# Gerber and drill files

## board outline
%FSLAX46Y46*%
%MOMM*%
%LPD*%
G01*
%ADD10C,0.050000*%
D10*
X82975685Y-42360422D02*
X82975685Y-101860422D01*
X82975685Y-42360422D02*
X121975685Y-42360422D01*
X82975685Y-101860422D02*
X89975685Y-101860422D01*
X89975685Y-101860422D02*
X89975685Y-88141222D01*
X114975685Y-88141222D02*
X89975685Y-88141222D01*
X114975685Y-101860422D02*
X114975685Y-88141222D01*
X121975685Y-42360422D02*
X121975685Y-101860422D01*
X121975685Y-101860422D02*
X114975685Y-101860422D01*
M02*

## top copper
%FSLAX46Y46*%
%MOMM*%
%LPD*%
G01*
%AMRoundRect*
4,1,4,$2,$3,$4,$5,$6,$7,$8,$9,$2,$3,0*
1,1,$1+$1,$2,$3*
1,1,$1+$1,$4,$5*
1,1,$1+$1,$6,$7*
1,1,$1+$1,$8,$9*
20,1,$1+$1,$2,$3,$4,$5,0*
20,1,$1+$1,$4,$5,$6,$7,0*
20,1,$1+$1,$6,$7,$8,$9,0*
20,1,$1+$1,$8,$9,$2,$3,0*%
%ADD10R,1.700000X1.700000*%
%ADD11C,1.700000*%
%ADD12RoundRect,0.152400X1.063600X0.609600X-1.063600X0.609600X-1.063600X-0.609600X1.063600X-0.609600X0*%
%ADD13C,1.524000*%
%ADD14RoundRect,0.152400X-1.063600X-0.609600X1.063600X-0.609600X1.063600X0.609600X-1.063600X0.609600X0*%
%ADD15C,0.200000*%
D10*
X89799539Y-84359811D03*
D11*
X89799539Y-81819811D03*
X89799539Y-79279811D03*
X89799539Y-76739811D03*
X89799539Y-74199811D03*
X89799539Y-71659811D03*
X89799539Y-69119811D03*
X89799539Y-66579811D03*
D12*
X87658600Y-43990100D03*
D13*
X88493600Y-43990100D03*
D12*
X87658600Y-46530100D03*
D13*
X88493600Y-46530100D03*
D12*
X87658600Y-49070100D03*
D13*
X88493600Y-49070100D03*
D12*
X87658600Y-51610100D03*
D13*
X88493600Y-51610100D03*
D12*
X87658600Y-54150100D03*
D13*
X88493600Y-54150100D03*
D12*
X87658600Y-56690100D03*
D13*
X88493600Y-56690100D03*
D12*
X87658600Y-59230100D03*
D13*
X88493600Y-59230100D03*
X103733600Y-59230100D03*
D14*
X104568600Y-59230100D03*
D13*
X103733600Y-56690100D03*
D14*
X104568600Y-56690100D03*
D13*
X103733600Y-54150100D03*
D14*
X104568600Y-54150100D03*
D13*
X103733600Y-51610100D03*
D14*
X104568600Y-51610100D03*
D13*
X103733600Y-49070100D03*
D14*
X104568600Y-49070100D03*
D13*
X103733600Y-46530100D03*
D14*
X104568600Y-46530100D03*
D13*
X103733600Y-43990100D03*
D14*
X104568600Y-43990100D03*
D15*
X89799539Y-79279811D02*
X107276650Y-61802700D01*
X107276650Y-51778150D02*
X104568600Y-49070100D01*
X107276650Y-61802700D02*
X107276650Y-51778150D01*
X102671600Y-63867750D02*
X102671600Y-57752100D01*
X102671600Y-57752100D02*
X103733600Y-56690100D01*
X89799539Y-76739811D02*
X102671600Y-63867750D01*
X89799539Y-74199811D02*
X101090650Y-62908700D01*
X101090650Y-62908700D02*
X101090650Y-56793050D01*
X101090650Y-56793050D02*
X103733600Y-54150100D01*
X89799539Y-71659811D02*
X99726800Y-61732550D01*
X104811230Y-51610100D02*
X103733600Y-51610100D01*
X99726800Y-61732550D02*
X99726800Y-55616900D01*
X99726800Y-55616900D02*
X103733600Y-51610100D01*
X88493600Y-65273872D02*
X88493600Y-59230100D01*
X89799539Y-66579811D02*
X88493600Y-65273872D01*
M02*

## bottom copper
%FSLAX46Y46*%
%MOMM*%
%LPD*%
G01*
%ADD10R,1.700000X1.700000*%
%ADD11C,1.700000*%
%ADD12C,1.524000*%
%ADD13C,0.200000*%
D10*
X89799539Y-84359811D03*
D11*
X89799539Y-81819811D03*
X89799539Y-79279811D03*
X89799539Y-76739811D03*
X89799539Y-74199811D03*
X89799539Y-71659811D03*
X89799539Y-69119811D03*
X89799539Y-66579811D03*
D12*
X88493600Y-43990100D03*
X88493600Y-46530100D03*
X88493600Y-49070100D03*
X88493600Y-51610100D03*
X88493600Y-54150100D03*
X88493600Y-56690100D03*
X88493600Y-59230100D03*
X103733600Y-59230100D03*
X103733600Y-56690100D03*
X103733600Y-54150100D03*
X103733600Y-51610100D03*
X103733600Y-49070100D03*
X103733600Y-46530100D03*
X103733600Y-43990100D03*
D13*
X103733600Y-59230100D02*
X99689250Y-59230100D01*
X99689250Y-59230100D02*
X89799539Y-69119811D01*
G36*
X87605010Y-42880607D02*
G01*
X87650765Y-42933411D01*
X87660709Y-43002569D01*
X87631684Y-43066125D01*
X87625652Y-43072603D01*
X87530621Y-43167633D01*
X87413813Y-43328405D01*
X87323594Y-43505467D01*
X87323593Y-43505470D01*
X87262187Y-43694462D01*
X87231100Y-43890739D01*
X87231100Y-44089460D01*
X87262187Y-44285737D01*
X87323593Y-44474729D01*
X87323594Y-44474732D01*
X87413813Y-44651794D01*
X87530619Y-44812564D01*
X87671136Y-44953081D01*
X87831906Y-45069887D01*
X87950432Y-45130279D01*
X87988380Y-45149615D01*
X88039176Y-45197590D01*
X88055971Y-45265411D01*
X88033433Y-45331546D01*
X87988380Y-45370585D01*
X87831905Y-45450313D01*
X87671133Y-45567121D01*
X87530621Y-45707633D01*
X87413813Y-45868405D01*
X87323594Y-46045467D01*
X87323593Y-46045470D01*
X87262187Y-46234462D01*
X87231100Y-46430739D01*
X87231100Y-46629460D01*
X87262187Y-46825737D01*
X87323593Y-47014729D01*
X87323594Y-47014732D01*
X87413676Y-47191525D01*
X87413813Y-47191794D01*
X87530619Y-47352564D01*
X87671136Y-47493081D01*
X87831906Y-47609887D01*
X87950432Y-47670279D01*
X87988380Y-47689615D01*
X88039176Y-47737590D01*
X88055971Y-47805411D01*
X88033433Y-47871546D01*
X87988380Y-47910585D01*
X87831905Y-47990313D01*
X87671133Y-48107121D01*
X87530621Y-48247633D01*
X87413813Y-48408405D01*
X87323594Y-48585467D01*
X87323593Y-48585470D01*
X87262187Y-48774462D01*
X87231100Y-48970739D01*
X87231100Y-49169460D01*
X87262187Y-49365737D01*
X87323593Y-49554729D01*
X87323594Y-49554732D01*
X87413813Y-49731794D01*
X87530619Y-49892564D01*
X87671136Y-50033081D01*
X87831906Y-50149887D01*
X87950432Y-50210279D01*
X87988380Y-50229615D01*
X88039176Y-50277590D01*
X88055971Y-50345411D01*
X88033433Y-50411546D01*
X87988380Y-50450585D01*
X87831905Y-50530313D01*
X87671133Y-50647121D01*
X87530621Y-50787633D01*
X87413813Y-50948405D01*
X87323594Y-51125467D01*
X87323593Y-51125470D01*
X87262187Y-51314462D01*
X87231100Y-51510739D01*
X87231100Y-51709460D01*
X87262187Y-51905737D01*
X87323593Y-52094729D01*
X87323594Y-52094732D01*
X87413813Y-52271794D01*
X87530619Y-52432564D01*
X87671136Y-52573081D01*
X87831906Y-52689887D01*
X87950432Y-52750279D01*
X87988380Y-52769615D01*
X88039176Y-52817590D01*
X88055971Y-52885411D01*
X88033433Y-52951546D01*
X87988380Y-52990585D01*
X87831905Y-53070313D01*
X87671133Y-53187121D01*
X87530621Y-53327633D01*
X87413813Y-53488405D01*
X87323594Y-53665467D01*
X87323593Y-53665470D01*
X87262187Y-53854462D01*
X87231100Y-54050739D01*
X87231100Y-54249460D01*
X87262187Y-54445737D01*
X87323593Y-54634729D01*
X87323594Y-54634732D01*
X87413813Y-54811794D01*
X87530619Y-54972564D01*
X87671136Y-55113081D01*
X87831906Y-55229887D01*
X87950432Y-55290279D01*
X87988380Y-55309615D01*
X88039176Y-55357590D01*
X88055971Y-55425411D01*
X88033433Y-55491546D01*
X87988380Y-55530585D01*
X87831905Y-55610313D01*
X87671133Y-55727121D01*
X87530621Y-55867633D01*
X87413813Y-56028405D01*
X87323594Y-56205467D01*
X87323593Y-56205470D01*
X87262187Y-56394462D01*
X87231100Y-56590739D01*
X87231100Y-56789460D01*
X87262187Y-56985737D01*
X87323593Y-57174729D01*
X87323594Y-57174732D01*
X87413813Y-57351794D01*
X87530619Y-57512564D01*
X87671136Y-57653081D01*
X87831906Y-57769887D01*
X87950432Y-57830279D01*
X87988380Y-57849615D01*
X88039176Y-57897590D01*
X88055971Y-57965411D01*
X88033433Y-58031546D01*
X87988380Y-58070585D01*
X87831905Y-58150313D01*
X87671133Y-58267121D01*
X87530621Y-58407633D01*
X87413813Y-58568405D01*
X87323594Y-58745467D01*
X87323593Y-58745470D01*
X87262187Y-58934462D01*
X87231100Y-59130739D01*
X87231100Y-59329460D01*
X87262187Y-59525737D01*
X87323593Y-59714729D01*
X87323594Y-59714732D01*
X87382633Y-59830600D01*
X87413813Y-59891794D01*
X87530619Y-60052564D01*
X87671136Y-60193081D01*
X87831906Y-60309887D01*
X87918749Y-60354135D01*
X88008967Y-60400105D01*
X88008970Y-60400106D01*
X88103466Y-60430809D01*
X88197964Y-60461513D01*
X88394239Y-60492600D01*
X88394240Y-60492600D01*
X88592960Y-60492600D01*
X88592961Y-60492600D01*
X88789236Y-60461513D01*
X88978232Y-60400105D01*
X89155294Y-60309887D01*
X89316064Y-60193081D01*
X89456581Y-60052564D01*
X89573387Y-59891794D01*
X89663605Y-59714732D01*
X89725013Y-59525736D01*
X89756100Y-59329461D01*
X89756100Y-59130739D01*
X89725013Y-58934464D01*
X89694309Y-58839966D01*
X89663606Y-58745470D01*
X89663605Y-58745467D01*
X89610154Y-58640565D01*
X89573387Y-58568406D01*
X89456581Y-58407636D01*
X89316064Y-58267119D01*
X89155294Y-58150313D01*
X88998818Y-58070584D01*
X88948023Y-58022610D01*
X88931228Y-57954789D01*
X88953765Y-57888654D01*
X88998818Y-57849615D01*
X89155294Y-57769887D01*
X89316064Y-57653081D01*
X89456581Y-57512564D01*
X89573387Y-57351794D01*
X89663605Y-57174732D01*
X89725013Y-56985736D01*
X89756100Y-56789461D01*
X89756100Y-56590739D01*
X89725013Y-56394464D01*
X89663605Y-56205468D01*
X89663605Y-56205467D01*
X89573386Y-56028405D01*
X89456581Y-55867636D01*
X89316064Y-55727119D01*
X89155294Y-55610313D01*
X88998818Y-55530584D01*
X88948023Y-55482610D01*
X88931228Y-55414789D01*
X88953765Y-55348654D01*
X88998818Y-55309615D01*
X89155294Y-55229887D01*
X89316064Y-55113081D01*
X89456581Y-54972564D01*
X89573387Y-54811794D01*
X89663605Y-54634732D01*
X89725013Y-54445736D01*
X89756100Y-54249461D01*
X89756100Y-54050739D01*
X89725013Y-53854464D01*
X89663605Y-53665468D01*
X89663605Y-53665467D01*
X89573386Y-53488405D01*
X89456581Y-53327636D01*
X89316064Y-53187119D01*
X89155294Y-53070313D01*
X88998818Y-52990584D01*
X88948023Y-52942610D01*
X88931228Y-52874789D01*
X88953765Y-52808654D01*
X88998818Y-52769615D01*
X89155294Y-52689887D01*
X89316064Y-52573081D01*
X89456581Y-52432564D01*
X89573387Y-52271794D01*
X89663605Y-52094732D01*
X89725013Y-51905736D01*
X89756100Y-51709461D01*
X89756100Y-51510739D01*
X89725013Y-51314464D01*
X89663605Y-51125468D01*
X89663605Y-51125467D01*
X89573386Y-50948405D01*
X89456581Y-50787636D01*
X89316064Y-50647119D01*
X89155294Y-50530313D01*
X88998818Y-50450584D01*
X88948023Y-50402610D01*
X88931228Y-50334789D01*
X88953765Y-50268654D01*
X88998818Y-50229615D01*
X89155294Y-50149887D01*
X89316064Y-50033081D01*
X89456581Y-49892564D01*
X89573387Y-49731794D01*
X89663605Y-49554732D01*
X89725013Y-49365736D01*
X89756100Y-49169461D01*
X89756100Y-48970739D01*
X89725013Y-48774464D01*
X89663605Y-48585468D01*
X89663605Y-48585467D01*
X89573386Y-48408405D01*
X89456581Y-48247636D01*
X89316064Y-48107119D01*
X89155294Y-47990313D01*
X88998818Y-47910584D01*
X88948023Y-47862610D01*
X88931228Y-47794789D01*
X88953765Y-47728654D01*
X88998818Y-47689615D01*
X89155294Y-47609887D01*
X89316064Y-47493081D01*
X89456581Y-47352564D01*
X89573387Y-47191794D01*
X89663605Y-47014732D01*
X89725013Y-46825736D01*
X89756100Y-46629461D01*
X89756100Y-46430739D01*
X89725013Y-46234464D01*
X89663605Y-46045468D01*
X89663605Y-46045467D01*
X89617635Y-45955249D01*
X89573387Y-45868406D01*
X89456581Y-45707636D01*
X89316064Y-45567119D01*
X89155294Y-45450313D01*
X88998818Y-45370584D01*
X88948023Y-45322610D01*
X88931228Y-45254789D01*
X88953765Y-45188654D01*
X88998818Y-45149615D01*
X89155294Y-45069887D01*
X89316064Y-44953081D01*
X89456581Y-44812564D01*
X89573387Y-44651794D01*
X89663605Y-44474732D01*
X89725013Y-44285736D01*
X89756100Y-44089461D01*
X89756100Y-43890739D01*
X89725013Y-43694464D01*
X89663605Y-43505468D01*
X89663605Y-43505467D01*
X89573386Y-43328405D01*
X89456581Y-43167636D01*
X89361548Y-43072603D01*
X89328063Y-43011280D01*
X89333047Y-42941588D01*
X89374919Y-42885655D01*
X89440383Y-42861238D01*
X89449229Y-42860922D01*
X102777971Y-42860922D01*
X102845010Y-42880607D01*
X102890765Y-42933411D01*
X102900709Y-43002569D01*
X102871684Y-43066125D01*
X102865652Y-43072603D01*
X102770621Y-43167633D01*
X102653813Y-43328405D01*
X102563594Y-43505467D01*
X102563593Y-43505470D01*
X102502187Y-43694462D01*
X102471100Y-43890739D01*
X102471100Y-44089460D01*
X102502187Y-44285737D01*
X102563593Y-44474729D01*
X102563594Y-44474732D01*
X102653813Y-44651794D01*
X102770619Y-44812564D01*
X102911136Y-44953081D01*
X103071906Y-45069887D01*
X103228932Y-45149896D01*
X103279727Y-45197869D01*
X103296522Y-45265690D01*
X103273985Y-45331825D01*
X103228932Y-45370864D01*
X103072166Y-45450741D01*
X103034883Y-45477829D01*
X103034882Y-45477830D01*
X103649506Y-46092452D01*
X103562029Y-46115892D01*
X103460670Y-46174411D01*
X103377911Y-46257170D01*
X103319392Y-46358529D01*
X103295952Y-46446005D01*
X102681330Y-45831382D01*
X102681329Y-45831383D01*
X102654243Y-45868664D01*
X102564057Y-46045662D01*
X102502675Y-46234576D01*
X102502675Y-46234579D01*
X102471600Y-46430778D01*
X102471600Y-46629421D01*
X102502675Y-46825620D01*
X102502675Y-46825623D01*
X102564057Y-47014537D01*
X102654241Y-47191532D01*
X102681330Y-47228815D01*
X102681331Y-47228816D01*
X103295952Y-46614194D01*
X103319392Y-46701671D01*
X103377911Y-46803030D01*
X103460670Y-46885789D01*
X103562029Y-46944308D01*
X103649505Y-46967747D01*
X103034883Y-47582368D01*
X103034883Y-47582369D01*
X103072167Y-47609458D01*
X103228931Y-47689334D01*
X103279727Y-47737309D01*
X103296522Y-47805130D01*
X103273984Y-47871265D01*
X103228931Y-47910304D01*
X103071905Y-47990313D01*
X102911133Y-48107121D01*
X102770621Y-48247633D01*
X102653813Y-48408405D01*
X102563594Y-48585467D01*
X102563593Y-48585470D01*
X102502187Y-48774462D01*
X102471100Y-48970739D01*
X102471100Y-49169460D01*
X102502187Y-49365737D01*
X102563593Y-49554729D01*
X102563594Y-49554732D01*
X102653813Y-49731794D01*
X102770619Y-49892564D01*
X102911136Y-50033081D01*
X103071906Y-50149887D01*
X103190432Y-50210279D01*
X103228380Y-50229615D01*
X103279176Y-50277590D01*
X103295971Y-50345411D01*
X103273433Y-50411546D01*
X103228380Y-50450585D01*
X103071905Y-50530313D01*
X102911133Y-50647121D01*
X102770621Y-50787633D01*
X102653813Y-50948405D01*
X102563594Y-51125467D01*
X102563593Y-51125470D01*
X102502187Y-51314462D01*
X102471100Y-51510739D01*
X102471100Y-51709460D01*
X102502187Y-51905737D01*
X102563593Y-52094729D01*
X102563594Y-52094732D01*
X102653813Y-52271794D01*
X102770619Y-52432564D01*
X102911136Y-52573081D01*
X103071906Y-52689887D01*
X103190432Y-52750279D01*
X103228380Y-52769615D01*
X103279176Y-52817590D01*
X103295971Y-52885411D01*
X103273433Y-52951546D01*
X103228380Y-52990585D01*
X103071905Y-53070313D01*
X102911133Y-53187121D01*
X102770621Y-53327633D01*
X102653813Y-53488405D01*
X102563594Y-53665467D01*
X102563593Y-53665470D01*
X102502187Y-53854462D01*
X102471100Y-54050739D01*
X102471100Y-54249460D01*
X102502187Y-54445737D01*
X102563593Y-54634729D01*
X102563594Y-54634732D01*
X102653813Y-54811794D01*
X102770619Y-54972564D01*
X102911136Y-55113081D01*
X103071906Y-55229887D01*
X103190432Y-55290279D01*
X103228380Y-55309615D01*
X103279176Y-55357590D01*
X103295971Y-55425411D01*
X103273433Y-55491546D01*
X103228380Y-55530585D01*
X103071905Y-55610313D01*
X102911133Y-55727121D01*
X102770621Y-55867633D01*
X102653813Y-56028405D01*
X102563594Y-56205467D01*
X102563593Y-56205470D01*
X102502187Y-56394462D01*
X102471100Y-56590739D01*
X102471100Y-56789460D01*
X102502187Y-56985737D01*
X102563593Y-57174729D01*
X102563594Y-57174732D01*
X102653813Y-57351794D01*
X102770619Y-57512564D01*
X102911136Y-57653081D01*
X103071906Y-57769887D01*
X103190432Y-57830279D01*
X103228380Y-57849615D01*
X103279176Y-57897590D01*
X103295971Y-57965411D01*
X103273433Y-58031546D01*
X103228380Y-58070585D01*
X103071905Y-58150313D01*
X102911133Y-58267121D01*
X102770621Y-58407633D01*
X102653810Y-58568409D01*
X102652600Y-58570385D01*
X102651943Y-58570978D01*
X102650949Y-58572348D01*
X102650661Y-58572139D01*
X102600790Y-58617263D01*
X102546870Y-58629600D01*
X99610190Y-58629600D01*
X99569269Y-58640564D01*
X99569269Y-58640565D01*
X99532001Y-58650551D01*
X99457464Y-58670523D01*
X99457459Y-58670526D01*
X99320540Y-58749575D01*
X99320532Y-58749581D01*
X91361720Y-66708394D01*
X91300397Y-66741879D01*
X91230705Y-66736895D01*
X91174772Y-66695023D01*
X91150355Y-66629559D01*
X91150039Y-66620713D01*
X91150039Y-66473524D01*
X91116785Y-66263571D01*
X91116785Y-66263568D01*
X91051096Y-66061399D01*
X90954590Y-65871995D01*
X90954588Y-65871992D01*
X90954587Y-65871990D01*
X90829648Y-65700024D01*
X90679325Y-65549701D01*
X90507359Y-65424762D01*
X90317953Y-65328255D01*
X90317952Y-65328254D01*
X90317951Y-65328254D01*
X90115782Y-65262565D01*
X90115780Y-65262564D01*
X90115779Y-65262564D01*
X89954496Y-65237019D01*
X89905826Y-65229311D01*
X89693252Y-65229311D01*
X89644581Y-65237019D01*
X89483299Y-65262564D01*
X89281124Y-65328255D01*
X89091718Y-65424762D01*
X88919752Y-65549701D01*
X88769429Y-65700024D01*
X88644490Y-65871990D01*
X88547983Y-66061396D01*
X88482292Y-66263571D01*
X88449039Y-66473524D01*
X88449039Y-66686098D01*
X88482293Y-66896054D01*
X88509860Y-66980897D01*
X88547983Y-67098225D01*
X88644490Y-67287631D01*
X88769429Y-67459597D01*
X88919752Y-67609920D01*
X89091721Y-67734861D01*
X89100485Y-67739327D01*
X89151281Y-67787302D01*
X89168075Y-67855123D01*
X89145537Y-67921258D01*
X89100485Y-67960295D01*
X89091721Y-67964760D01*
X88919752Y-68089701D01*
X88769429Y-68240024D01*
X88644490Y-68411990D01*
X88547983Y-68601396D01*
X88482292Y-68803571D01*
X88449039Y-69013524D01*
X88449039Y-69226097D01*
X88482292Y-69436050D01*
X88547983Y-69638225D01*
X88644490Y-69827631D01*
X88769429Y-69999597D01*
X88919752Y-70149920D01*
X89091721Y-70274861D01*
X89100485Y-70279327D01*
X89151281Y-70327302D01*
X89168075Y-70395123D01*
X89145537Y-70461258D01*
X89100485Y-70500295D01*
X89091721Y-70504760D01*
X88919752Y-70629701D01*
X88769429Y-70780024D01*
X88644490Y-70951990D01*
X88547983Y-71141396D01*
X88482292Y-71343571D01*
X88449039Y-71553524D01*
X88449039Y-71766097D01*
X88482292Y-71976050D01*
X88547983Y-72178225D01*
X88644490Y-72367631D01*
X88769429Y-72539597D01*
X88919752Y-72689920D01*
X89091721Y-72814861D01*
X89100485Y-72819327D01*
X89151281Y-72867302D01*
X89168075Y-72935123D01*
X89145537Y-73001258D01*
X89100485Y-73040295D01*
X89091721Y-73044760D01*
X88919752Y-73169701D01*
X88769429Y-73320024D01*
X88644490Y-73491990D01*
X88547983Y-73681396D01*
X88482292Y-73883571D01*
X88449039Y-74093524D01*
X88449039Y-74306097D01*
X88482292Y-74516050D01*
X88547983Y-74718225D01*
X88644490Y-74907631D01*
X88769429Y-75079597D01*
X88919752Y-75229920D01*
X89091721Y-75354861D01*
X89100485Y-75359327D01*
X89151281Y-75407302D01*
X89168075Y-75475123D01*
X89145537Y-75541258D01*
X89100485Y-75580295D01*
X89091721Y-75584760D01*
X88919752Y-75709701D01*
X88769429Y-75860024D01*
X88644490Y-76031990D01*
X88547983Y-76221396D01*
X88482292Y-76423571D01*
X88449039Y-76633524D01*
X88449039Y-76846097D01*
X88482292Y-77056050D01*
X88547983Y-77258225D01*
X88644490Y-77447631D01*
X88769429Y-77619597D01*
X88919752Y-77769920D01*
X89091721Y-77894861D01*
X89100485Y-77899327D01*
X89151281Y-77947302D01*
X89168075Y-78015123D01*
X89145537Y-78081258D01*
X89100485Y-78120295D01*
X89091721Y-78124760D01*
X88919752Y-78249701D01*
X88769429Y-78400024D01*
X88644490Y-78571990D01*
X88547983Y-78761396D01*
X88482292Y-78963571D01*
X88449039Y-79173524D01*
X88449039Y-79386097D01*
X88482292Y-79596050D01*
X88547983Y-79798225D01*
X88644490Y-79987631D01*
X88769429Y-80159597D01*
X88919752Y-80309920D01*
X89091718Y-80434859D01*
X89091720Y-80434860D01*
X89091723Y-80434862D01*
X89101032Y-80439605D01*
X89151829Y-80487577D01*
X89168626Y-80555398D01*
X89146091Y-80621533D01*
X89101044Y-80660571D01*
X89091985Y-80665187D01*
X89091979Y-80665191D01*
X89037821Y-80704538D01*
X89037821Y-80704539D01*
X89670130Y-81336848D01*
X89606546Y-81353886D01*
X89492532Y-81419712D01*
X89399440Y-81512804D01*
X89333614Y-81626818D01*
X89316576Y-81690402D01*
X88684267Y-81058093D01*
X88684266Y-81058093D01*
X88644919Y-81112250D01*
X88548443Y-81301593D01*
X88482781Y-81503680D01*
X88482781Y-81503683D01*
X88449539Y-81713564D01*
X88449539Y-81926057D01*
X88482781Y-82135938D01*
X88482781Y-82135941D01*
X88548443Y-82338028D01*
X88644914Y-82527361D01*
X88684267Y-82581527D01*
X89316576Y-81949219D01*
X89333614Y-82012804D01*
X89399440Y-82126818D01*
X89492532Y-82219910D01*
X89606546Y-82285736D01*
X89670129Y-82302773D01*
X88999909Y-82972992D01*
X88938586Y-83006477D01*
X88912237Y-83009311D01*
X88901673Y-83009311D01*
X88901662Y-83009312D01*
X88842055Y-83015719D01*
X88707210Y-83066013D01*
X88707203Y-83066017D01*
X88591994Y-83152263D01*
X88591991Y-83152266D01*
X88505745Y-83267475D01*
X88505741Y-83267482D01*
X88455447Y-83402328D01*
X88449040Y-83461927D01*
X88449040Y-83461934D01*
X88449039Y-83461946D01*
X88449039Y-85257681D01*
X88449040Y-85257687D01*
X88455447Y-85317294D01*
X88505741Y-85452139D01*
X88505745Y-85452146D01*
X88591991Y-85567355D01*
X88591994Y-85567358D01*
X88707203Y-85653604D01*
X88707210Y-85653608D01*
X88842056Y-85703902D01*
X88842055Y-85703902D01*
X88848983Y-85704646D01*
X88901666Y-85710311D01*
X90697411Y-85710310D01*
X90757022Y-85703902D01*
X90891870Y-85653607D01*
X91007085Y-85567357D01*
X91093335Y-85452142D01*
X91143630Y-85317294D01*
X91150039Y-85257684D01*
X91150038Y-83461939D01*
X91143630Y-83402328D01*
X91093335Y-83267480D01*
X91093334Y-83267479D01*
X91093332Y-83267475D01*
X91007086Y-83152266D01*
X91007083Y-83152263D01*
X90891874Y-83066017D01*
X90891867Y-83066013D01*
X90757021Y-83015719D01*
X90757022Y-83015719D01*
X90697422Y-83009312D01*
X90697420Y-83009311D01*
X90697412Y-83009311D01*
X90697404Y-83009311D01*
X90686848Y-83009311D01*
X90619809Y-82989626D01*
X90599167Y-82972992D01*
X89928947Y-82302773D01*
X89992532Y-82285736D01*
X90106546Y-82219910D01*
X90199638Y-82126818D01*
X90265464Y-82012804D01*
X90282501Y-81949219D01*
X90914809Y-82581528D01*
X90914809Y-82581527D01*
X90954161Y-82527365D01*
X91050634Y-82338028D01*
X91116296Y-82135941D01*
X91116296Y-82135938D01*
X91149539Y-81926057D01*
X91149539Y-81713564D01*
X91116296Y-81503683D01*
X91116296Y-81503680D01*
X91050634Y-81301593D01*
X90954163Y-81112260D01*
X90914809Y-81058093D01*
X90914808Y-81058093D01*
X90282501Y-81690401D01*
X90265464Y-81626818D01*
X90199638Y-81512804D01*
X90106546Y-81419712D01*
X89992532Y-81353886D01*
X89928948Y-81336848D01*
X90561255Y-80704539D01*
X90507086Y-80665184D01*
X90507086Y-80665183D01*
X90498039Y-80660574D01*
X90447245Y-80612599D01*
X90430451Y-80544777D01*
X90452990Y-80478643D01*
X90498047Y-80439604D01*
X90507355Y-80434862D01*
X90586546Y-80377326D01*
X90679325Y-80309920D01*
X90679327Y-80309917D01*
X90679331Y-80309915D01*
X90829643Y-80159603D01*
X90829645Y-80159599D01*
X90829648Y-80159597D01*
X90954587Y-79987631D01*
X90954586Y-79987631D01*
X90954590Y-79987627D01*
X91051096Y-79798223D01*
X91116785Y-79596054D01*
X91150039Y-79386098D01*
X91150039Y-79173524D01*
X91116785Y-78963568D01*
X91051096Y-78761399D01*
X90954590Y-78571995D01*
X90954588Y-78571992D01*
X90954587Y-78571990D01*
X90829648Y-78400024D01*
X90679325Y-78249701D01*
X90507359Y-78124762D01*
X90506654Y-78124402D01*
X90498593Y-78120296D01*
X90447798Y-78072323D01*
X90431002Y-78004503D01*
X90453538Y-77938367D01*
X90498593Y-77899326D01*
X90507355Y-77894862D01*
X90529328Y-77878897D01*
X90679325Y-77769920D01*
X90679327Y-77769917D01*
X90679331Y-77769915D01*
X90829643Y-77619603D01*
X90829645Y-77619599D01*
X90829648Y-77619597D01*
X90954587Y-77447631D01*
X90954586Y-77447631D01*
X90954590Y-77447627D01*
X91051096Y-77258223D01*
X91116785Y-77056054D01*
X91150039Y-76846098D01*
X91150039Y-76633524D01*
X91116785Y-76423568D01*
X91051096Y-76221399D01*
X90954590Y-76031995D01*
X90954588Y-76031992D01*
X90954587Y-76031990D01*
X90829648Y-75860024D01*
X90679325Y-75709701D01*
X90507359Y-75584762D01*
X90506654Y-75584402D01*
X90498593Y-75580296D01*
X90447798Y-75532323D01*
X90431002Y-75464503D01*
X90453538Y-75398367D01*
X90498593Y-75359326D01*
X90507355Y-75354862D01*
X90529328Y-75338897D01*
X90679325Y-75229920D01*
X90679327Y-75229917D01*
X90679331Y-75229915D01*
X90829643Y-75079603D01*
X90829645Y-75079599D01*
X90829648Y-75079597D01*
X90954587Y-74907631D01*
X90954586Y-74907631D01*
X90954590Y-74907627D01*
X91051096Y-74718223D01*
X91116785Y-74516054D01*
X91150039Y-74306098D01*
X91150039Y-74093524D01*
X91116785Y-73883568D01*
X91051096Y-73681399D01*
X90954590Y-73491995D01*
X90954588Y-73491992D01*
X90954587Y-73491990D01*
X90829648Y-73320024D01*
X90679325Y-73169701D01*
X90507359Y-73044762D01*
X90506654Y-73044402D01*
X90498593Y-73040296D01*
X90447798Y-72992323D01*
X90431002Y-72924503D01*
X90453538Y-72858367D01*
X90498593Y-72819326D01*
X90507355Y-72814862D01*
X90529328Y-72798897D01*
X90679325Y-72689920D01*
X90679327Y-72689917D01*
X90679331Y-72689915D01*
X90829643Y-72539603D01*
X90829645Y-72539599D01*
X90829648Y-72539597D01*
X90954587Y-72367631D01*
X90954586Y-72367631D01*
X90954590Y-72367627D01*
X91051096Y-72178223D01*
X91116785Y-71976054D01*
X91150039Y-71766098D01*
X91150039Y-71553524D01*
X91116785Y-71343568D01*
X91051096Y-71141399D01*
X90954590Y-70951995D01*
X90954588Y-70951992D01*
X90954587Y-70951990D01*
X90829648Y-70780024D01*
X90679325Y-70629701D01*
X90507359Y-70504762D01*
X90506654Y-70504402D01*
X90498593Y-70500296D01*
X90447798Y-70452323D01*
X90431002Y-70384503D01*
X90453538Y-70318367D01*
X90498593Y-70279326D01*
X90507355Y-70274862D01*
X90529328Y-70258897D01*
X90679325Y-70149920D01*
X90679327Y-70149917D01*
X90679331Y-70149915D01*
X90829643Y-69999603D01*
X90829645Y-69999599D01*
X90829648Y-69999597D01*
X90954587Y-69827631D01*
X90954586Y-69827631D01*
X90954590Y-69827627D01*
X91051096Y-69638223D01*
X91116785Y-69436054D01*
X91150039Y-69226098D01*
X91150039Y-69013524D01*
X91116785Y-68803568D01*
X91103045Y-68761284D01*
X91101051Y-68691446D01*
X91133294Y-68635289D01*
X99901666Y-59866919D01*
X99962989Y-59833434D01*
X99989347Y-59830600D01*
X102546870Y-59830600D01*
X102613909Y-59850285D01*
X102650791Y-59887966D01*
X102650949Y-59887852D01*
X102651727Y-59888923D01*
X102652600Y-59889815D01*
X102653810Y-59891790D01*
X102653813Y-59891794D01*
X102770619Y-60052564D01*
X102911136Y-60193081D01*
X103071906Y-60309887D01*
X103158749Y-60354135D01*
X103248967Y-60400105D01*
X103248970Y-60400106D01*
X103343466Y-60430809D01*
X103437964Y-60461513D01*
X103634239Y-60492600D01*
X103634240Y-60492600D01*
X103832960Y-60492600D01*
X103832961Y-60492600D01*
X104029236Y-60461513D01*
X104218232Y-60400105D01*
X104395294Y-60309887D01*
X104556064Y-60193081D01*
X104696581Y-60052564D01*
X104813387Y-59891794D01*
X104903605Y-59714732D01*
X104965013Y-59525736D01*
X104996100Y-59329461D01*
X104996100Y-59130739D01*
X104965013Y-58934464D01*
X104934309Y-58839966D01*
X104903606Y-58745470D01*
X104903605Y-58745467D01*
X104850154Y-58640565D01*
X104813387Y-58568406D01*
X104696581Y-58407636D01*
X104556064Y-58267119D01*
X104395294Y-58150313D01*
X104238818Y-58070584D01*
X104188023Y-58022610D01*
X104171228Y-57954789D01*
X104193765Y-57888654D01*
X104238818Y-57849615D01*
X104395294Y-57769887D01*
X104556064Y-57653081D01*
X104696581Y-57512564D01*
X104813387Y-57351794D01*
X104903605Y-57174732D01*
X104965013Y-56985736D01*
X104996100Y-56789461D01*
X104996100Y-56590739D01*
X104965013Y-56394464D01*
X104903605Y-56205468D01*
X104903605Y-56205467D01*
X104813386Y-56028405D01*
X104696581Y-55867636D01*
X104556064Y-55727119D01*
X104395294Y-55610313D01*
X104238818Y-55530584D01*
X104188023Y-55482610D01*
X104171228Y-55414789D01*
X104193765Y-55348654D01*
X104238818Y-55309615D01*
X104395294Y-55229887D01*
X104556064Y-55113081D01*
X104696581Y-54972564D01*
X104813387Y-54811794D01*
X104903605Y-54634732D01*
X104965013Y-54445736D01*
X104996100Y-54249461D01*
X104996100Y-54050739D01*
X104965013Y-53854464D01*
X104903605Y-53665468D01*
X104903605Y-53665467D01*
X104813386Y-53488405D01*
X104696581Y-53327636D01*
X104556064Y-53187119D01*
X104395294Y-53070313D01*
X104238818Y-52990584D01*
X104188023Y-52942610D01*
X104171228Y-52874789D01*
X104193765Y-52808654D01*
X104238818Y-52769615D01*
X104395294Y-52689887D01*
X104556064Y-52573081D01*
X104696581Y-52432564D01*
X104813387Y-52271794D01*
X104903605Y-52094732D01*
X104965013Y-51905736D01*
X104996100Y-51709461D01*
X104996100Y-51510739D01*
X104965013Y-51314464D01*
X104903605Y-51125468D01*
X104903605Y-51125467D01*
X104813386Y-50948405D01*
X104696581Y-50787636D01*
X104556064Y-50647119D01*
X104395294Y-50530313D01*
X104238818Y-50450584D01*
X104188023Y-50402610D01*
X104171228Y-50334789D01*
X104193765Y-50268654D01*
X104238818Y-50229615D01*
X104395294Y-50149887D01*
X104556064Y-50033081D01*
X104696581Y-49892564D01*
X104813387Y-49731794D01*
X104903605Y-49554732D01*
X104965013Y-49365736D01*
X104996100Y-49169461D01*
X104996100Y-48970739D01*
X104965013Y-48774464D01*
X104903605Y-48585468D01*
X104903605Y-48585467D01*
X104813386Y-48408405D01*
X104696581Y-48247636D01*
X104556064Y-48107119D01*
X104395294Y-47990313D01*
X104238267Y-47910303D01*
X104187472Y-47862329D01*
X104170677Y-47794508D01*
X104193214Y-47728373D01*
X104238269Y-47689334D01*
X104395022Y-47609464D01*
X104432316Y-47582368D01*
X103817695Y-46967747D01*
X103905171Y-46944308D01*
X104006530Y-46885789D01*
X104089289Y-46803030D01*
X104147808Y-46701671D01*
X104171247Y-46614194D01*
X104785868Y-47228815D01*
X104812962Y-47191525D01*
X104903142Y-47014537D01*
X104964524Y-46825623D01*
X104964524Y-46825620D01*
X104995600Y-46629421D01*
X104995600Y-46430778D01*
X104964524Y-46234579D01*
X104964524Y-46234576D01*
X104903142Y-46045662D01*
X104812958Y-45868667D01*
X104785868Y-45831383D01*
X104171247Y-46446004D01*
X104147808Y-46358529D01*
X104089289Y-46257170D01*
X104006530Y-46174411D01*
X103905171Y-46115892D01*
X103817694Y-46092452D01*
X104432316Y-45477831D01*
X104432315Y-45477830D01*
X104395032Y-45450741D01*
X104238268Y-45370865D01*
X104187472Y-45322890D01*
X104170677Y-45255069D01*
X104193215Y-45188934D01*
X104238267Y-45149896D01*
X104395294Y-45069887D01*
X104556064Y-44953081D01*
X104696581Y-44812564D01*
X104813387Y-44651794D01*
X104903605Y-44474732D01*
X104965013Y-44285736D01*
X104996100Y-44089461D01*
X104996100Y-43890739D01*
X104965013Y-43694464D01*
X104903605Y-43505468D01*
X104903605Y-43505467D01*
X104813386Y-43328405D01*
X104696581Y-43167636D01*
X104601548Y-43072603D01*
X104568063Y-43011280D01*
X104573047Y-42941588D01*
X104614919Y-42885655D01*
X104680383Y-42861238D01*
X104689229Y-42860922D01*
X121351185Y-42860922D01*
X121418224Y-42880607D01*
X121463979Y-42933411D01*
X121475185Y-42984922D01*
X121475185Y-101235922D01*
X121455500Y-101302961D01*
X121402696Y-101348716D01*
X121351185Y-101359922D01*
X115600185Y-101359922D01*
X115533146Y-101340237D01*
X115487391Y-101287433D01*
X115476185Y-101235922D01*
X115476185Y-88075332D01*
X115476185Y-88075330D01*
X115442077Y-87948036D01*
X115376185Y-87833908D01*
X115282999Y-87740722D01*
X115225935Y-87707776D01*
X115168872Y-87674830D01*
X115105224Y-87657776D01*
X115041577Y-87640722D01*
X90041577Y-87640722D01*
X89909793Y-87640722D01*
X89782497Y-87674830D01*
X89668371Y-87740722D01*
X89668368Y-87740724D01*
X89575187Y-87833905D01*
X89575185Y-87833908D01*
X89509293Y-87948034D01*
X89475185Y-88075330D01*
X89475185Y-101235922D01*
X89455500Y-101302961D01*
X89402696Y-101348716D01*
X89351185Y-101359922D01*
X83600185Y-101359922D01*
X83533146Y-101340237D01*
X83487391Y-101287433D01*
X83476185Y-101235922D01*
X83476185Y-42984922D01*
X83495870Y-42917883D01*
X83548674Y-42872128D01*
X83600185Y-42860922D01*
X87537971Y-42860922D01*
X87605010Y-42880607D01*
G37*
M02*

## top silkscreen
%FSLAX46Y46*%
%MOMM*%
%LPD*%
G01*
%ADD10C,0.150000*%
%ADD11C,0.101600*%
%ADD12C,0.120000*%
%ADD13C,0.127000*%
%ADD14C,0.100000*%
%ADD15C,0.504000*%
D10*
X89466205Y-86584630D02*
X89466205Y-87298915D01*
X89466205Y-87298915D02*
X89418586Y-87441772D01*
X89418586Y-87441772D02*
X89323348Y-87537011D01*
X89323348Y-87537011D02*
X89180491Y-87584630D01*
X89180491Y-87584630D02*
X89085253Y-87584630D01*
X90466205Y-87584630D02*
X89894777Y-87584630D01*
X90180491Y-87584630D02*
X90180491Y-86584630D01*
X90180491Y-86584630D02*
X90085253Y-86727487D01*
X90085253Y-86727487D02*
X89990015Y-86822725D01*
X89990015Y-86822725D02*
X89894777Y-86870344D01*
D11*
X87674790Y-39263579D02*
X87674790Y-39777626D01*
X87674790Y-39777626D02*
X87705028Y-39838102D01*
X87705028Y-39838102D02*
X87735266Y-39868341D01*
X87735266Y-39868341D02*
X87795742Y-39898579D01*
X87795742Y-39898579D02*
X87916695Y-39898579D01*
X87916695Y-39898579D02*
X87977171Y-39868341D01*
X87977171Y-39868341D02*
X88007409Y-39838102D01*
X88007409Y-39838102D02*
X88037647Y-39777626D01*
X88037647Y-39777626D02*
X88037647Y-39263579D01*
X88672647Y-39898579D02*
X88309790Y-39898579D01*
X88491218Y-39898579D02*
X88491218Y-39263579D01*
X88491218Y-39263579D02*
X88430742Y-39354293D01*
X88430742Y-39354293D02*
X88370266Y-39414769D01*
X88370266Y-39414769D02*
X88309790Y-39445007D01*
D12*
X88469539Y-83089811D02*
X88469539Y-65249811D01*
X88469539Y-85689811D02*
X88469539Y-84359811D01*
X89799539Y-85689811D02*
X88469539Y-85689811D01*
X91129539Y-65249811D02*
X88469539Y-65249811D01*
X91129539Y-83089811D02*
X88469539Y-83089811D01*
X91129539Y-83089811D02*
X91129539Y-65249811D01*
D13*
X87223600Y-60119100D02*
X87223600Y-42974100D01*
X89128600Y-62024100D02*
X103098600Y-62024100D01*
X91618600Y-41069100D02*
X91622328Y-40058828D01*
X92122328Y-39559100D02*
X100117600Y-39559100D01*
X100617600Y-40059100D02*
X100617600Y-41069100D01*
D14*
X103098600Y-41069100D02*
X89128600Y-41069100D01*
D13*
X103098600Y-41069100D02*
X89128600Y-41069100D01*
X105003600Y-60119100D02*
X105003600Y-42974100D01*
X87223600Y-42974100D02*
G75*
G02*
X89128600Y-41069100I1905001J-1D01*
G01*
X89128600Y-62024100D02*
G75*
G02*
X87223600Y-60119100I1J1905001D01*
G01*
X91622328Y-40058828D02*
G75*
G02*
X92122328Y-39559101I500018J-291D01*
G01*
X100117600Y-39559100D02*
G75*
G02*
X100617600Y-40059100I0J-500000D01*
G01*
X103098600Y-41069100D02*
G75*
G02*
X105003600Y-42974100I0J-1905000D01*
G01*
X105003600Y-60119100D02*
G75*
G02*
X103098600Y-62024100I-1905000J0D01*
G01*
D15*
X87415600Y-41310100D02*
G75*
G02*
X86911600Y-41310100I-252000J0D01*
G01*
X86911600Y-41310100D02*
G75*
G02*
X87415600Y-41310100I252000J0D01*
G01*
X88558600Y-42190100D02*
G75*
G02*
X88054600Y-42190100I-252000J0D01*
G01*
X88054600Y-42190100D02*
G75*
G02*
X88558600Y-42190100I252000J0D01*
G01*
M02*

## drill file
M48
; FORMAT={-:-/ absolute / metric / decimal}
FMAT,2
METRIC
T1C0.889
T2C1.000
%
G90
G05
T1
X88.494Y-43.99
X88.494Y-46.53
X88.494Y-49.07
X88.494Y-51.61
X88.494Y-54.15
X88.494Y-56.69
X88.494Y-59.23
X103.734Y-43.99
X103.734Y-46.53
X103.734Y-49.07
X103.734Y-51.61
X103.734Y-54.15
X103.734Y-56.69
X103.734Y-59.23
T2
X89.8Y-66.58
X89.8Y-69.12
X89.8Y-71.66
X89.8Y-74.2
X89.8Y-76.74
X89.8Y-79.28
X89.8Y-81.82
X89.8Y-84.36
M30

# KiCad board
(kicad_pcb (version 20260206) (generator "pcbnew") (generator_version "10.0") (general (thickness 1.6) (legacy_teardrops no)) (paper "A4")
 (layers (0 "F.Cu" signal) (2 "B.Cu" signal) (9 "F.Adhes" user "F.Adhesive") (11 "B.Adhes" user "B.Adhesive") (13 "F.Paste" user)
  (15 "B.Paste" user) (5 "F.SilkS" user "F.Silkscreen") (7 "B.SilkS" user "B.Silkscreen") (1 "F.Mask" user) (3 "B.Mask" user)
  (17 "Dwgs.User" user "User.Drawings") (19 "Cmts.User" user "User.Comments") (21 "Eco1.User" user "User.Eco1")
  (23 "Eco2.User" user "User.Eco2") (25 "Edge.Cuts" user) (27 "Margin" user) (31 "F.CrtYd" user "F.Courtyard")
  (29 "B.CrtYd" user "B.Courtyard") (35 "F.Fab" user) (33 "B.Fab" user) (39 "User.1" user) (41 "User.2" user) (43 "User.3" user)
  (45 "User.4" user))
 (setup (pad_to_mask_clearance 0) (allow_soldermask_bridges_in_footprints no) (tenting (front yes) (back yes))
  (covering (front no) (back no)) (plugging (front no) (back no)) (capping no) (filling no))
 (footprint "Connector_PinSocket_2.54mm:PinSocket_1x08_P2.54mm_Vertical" (layer "F.Cu") (at 89.799539 84.359811 180)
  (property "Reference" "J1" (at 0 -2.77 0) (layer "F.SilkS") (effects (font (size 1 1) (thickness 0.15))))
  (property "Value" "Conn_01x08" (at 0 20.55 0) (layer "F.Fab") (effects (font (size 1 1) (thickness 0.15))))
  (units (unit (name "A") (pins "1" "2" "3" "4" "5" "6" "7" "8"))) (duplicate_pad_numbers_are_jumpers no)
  (fp_line (start 1.33 1.27) (end 1.33 19.11) (stroke (width 0.12) (type solid)) (layer "F.SilkS"))
  (fp_line (start 1.33 -1.33) (end 1.33 0) (stroke (width 0.12) (type solid)) (layer "F.SilkS"))
  (fp_line (start 0 -1.33) (end 1.33 -1.33) (stroke (width 0.12) (type solid)) (layer "F.SilkS"))
  (fp_line (start -1.33 19.11) (end 1.33 19.11) (stroke (width 0.12) (type solid)) (layer "F.SilkS"))
  (fp_line (start -1.33 1.27) (end 1.33 1.27) (stroke (width 0.12) (type solid)) (layer "F.SilkS"))
  (fp_line (start -1.33 1.27) (end -1.33 19.11) (stroke (width 0.12) (type solid)) (layer "F.SilkS"))
  (pad "1" thru_hole rect (at 0 0 180) (size 1.7 1.7) (drill 1) (layers "*.Cu" "*.Mask") (remove_unused_layers no) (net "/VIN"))
  (pad "2" thru_hole circle (at 0 2.54 180) (size 1.7 1.7) (drill 1) (layers "*.Cu" "*.Mask") (remove_unused_layers no) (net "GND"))
  (pad "3" thru_hole circle (at 0 5.08 180) (size 1.7 1.7) (drill 1) (layers "*.Cu" "*.Mask") (remove_unused_layers no) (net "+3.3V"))
  (pad "4" thru_hole circle (at 0 7.62 180) (size 1.7 1.7) (drill 1) (layers "*.Cu" "*.Mask") (remove_unused_layers no) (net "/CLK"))
  (pad "5" thru_hole circle (at 0 10.16 180) (size 1.7 1.7) (drill 1) (layers "*.Cu" "*.Mask") (remove_unused_layers no) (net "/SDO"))
  (pad "6" thru_hole circle (at 0 12.7 180) (size 1.7 1.7) (drill 1) (layers "*.Cu" "*.Mask") (remove_unused_layers no) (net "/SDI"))
  (pad "7" thru_hole circle (at 0 15.24 180) (size 1.7 1.7) (drill 1) (layers "*.Cu" "*.Mask") (remove_unused_layers no) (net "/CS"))
  (pad "8" thru_hole circle (at 0 17.78 180) (size 1.7 1.7) (drill 1) (layers "*.Cu" "*.Mask") (remove_unused_layers no) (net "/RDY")))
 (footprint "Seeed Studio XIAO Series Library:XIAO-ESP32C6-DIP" (layer "F.Cu") (at 96.1586 51.6101)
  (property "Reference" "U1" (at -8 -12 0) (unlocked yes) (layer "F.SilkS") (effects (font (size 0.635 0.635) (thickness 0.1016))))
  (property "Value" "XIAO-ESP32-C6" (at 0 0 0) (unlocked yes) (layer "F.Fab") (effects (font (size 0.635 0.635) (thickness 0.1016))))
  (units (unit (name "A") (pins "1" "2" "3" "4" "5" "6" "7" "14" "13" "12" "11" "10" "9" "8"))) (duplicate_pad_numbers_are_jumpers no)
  (fp_line (start -8.935 8.509) (end -8.935 -8.636) (stroke (width 0.127) (type solid)) (layer "F.SilkS"))
  (fp_line (start -7.03 10.414) (end 6.94 10.414) (stroke (width 0.127) (type solid)) (layer "F.SilkS"))
  (fp_line (start -4.54 -10.541) (end -4.536272 -11.551272) (stroke (width 0.127) (type solid)) (layer "F.SilkS"))
  (fp_line (start -4.036272 -12.051) (end 3.959 -12.051) (stroke (width 0.127) (type solid)) (layer "F.SilkS"))
  (fp_line (start 4.459 -11.551) (end 4.459 -10.541) (stroke (width 0.127) (type solid)) (layer "F.SilkS"))
  (fp_line (start 6.94 -10.541) (end -7.03 -10.541) (stroke (width 0.1) (type solid)) (layer "F.SilkS"))
  (fp_line (start 6.94 -10.541) (end -7.03 -10.541) (stroke (width 0.127) (type solid)) (layer "F.SilkS"))
  (fp_line (start 8.845 8.509) (end 8.845 -8.636) (stroke (width 0.127) (type solid)) (layer "F.SilkS"))
  (fp_arc (start -8.935 -8.636) (mid -8.377038 -9.983038) (end -7.03 -10.541) (stroke (width 0.127) (type solid)) (layer "F.SilkS"))
  (fp_arc (start -7.03 10.414) (mid -8.377038 9.856038) (end -8.935 8.509) (stroke (width 0.127) (type solid)) (layer "F.SilkS"))
  (fp_arc (start -4.536272 -11.551272) (mid -4.389728 -11.90464) (end -4.036272 -12.051) (stroke (width 0.127) (type default))
   (layer "F.SilkS"))
  (fp_arc (start 3.959 -12.051) (mid 4.312553 -11.904553) (end 4.459 -11.551) (stroke (width 0.127) (type default)) (layer "F.SilkS"))
  (fp_arc (start 6.94 -10.541) (mid 8.287038 -9.983038) (end 8.845 -8.636) (stroke (width 0.127) (type solid)) (layer "F.SilkS"))
  (fp_arc (start 8.845 8.509) (mid 8.287038 9.856038) (end 6.94 10.414) (stroke (width 0.127) (type solid)) (layer "F.SilkS"))
  (fp_circle (center -8.995 -10.3) (end -8.995 -10.554) (stroke (width 0.5) (type solid)) (fill yes) (layer "F.SilkS"))
  (fp_circle (center -7.852 -9.42) (end -7.852 -9.674) (stroke (width 0.5) (type solid)) (fill yes) (layer "F.SilkS"))
  (pad "1" smd roundrect (at -8.5 -7.62 180) (size 2.432 1.524) (layers "F.Cu" "F.Mask") (roundrect_rratio 0.1)
   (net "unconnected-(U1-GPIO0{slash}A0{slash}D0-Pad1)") (thermal_bridge_angle 45))
  (pad "1" thru_hole circle (at -7.665 -7.62 180) (size 1.524 1.524) (drill 0.889) (layers "*.Cu" "*.Mask") (remove_unused_layers no)
   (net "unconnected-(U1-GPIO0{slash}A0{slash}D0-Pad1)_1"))
  (pad "2" smd roundrect (at -8.5 -5.08 180) (size 2.432 1.524) (layers "F.Cu" "F.Mask") (roundrect_rratio 0.1)
   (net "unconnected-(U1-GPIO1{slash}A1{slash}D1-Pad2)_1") (thermal_bridge_angle 45))
  (pad "2" thru_hole circle (at -7.665 -5.08 180) (size 1.524 1.524) (drill 0.889) (layers "*.Cu" "*.Mask") (remove_unused_layers no)
   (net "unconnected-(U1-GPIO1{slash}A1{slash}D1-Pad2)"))
  (pad "3" smd roundrect (at -8.5 -2.54 180) (size 2.432 1.524) (layers "F.Cu" "F.Mask") (roundrect_rratio 0.1)
   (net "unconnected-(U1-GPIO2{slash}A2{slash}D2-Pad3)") (thermal_bridge_angle 45))
  (pad "3" thru_hole circle (at -7.665 -2.54 180) (size 1.524 1.524) (drill 0.889) (layers "*.Cu" "*.Mask") (remove_unused_layers no)
   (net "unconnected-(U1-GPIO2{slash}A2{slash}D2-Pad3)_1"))
  (pad "4" smd roundrect (at -8.5 0 180) (size 2.432 1.524) (layers "F.Cu" "F.Mask") (roundrect_rratio 0.1)
   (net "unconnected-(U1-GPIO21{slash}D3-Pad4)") (thermal_bridge_angle 45))
  (pad "4" thru_hole circle (at -7.665 0 180) (size 1.524 1.524) (drill 0.889) (layers "*.Cu" "*.Mask") (remove_unused_layers no)
   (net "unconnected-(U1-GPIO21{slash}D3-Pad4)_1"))
  (pad "5" smd roundrect (at -8.5 2.54 180) (size 2.432 1.524) (layers "F.Cu" "F.Mask") (roundrect_rratio 0.1)
   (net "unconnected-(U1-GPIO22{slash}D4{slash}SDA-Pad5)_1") (thermal_bridge_angle 45))
  (pad "5" thru_hole circle (at -7.665 2.54 180) (size 1.524 1.524) (drill 0.889) (layers "*.Cu" "*.Mask") (remove_unused_layers no)
   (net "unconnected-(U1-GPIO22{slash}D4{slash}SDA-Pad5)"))
  (pad "6" smd roundrect (at -8.5 5.08 180) (size 2.432 1.524) (layers "F.Cu" "F.Mask") (roundrect_rratio 0.1)
   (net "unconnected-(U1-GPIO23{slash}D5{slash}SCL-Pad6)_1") (thermal_bridge_angle 45))
  (pad "6" thru_hole circle (at -7.665 5.08 180) (size 1.524 1.524) (drill 0.889) (layers "*.Cu" "*.Mask") (remove_unused_layers no)
   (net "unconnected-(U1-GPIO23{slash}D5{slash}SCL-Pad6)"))
  (pad "7" smd roundrect (at -8.5 7.62 180) (size 2.432 1.524) (layers "F.Cu" "F.Mask") (roundrect_rratio 0.1) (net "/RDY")
   (thermal_bridge_angle 45))
  (pad "7" thru_hole circle (at -7.665 7.62 180) (size 1.524 1.524) (drill 0.889) (layers "*.Cu" "*.Mask") (remove_unused_layers no)
   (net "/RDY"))
  (pad "8" thru_hole circle (at 7.575 7.62) (size 1.524 1.524) (drill 0.889) (layers "*.Cu" "*.Mask") (remove_unused_layers no) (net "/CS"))
  (pad "8" smd roundrect (at 8.41 7.62) (size 2.432 1.524) (layers "F.Cu" "F.Mask") (roundrect_rratio 0.1) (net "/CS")
   (thermal_bridge_angle 45))
  (pad "9" thru_hole circle (at 7.575 5.08) (size 1.524 1.524) (drill 0.889) (layers "*.Cu" "*.Mask") (remove_unused_layers no) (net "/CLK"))
  (pad "9" smd roundrect (at 8.41 5.08) (size 2.432 1.524) (layers "F.Cu" "F.Mask") (roundrect_rratio 0.1) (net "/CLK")
   (thermal_bridge_angle 45))
  (pad "10" thru_hole circle (at 7.575 2.54) (size 1.524 1.524) (drill 0.889) (layers "*.Cu" "*.Mask") (remove_unused_layers no)
   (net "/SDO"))
  (pad "10" smd roundrect (at 8.41 2.54) (size 2.432 1.524) (layers "F.Cu" "F.Mask") (roundrect_rratio 0.1) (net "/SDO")
   (thermal_bridge_angle 45))
  (pad "11" thru_hole circle (at 7.575 0) (size 1.524 1.524) (drill 0.889) (layers "*.Cu" "*.Mask") (remove_unused_layers no) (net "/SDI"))
  (pad "11" smd roundrect (at 8.41 0) (size 2.432 1.524) (layers "F.Cu" "F.Mask") (roundrect_rratio 0.1) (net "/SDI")
   (thermal_bridge_angle 45))
  (pad "12" thru_hole circle (at 7.575 -2.54) (size 1.524 1.524) (drill 0.889) (layers "*.Cu" "*.Mask") (remove_unused_layers no)
   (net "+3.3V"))
  (pad "12" smd roundrect (at 8.41 -2.54) (size 2.432 1.524) (layers "F.Cu" "F.Mask") (roundrect_rratio 0.1) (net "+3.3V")
   (thermal_bridge_angle 45))
  (pad "13" thru_hole circle (at 7.575 -5.08) (size 1.524 1.524) (drill 0.889) (layers "*.Cu" "*.Mask") (remove_unused_layers no)
   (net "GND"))
  (pad "13" smd roundrect (at 8.41 -5.08) (size 2.432 1.524) (layers "F.Cu" "F.Mask") (roundrect_rratio 0.1) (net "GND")
   (thermal_bridge_angle 45))
  (pad "14" thru_hole circle (at 7.575 -7.62) (size 1.524 1.524) (drill 0.889) (layers "*.Cu" "*.Mask") (remove_unused_layers no)
   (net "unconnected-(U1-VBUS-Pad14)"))
  (pad "14" smd roundrect (at 8.41 -7.62) (size 2.432 1.524) (layers "F.Cu" "F.Mask") (roundrect_rratio 0.1)
   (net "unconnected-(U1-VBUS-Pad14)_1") (thermal_bridge_angle 45)))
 (gr_line (start 82.975685 42.360422) (end 82.975685 101.860422) (stroke (width 0.05) (type solid)) (layer "Edge.Cuts"))
 (gr_line (start 82.975685 42.360422) (end 121.975685 42.360422) (stroke (width 0.05) (type default)) (layer "Edge.Cuts"))
 (gr_line (start 82.975685 101.860422) (end 89.975685 101.860422) (stroke (width 0.05) (type solid)) (layer "Edge.Cuts"))
 (gr_line (start 89.975685 101.860422) (end 89.975685 88.141222) (stroke (width 0.05) (type solid)) (layer "Edge.Cuts"))
 (gr_line (start 114.975685 88.141222) (end 89.975685 88.141222) (stroke (width 0.05) (type default)) (layer "Edge.Cuts"))
 (gr_line (start 114.975685 101.860422) (end 114.975685 88.141222) (stroke (width 0.05) (type solid)) (layer "Edge.Cuts"))
 (gr_line (start 121.975685 42.360422) (end 121.975685 101.860422) (stroke (width 0.05) (type solid)) (layer "Edge.Cuts"))
 (gr_line (start 121.975685 101.860422) (end 114.975685 101.860422) (stroke (width 0.05) (type solid)) (layer "Edge.Cuts"))
 (segment (start 89.799539 79.279811) (end 107.27665 61.8027) (width 0.2) (layer "F.Cu") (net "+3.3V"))
 (segment (start 107.27665 51.77815) (end 104.5686 49.0701) (width 0.2) (layer "F.Cu") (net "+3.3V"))
 (segment (start 107.27665 61.8027) (end 107.27665 51.77815) (width 0.2) (layer "F.Cu") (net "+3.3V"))
 (segment (start 102.6716 63.86775) (end 102.6716 57.7521) (width 0.2) (layer "F.Cu") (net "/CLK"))
 (segment (start 102.6716 57.7521) (end 103.7336 56.6901) (width 0.2) (layer "F.Cu") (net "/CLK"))
 (segment (start 89.799539 76.739811) (end 102.6716 63.86775) (width 0.2) (layer "F.Cu") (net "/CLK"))
 (segment (start 89.799539 74.199811) (end 101.09065 62.9087) (width 0.2) (layer "F.Cu") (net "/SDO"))
 (segment (start 101.09065 62.9087) (end 101.09065 56.79305) (width 0.2) (layer "F.Cu") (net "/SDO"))
 (segment (start 101.09065 56.79305) (end 103.7336 54.1501) (width 0.2) (layer "F.Cu") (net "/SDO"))
 (segment (start 89.799539 71.659811) (end 99.7268 61.73255) (width 0.2) (layer "F.Cu") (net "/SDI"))
 (segment (start 104.81123 51.6101) (end 103.7336 51.6101) (width 0.2) (layer "F.Cu") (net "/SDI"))
 (segment (start 99.7268 61.73255) (end 99.7268 55.6169) (width 0.2) (layer "F.Cu") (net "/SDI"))
 (segment (start 99.7268 55.6169) (end 103.7336 51.6101) (width 0.2) (layer "F.Cu") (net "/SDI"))
 (segment (start 103.7336 59.2301) (end 99.68925 59.2301) (width 0.2) (layer "B.Cu") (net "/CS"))
 (segment (start 99.68925 59.2301) (end 89.799539 69.119811) (width 0.2) (layer "B.Cu") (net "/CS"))
 (segment (start 88.4936 65.273872) (end 88.4936 59.2301) (width 0.2) (layer "F.Cu") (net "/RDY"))
 (segment (start 89.799539 66.579811) (end 88.4936 65.273872) (width 0.2) (layer "F.Cu") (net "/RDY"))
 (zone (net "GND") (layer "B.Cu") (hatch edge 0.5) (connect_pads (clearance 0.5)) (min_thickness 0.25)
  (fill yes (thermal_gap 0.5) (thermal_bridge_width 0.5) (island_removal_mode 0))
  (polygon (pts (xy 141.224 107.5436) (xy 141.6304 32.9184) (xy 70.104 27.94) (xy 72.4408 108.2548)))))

